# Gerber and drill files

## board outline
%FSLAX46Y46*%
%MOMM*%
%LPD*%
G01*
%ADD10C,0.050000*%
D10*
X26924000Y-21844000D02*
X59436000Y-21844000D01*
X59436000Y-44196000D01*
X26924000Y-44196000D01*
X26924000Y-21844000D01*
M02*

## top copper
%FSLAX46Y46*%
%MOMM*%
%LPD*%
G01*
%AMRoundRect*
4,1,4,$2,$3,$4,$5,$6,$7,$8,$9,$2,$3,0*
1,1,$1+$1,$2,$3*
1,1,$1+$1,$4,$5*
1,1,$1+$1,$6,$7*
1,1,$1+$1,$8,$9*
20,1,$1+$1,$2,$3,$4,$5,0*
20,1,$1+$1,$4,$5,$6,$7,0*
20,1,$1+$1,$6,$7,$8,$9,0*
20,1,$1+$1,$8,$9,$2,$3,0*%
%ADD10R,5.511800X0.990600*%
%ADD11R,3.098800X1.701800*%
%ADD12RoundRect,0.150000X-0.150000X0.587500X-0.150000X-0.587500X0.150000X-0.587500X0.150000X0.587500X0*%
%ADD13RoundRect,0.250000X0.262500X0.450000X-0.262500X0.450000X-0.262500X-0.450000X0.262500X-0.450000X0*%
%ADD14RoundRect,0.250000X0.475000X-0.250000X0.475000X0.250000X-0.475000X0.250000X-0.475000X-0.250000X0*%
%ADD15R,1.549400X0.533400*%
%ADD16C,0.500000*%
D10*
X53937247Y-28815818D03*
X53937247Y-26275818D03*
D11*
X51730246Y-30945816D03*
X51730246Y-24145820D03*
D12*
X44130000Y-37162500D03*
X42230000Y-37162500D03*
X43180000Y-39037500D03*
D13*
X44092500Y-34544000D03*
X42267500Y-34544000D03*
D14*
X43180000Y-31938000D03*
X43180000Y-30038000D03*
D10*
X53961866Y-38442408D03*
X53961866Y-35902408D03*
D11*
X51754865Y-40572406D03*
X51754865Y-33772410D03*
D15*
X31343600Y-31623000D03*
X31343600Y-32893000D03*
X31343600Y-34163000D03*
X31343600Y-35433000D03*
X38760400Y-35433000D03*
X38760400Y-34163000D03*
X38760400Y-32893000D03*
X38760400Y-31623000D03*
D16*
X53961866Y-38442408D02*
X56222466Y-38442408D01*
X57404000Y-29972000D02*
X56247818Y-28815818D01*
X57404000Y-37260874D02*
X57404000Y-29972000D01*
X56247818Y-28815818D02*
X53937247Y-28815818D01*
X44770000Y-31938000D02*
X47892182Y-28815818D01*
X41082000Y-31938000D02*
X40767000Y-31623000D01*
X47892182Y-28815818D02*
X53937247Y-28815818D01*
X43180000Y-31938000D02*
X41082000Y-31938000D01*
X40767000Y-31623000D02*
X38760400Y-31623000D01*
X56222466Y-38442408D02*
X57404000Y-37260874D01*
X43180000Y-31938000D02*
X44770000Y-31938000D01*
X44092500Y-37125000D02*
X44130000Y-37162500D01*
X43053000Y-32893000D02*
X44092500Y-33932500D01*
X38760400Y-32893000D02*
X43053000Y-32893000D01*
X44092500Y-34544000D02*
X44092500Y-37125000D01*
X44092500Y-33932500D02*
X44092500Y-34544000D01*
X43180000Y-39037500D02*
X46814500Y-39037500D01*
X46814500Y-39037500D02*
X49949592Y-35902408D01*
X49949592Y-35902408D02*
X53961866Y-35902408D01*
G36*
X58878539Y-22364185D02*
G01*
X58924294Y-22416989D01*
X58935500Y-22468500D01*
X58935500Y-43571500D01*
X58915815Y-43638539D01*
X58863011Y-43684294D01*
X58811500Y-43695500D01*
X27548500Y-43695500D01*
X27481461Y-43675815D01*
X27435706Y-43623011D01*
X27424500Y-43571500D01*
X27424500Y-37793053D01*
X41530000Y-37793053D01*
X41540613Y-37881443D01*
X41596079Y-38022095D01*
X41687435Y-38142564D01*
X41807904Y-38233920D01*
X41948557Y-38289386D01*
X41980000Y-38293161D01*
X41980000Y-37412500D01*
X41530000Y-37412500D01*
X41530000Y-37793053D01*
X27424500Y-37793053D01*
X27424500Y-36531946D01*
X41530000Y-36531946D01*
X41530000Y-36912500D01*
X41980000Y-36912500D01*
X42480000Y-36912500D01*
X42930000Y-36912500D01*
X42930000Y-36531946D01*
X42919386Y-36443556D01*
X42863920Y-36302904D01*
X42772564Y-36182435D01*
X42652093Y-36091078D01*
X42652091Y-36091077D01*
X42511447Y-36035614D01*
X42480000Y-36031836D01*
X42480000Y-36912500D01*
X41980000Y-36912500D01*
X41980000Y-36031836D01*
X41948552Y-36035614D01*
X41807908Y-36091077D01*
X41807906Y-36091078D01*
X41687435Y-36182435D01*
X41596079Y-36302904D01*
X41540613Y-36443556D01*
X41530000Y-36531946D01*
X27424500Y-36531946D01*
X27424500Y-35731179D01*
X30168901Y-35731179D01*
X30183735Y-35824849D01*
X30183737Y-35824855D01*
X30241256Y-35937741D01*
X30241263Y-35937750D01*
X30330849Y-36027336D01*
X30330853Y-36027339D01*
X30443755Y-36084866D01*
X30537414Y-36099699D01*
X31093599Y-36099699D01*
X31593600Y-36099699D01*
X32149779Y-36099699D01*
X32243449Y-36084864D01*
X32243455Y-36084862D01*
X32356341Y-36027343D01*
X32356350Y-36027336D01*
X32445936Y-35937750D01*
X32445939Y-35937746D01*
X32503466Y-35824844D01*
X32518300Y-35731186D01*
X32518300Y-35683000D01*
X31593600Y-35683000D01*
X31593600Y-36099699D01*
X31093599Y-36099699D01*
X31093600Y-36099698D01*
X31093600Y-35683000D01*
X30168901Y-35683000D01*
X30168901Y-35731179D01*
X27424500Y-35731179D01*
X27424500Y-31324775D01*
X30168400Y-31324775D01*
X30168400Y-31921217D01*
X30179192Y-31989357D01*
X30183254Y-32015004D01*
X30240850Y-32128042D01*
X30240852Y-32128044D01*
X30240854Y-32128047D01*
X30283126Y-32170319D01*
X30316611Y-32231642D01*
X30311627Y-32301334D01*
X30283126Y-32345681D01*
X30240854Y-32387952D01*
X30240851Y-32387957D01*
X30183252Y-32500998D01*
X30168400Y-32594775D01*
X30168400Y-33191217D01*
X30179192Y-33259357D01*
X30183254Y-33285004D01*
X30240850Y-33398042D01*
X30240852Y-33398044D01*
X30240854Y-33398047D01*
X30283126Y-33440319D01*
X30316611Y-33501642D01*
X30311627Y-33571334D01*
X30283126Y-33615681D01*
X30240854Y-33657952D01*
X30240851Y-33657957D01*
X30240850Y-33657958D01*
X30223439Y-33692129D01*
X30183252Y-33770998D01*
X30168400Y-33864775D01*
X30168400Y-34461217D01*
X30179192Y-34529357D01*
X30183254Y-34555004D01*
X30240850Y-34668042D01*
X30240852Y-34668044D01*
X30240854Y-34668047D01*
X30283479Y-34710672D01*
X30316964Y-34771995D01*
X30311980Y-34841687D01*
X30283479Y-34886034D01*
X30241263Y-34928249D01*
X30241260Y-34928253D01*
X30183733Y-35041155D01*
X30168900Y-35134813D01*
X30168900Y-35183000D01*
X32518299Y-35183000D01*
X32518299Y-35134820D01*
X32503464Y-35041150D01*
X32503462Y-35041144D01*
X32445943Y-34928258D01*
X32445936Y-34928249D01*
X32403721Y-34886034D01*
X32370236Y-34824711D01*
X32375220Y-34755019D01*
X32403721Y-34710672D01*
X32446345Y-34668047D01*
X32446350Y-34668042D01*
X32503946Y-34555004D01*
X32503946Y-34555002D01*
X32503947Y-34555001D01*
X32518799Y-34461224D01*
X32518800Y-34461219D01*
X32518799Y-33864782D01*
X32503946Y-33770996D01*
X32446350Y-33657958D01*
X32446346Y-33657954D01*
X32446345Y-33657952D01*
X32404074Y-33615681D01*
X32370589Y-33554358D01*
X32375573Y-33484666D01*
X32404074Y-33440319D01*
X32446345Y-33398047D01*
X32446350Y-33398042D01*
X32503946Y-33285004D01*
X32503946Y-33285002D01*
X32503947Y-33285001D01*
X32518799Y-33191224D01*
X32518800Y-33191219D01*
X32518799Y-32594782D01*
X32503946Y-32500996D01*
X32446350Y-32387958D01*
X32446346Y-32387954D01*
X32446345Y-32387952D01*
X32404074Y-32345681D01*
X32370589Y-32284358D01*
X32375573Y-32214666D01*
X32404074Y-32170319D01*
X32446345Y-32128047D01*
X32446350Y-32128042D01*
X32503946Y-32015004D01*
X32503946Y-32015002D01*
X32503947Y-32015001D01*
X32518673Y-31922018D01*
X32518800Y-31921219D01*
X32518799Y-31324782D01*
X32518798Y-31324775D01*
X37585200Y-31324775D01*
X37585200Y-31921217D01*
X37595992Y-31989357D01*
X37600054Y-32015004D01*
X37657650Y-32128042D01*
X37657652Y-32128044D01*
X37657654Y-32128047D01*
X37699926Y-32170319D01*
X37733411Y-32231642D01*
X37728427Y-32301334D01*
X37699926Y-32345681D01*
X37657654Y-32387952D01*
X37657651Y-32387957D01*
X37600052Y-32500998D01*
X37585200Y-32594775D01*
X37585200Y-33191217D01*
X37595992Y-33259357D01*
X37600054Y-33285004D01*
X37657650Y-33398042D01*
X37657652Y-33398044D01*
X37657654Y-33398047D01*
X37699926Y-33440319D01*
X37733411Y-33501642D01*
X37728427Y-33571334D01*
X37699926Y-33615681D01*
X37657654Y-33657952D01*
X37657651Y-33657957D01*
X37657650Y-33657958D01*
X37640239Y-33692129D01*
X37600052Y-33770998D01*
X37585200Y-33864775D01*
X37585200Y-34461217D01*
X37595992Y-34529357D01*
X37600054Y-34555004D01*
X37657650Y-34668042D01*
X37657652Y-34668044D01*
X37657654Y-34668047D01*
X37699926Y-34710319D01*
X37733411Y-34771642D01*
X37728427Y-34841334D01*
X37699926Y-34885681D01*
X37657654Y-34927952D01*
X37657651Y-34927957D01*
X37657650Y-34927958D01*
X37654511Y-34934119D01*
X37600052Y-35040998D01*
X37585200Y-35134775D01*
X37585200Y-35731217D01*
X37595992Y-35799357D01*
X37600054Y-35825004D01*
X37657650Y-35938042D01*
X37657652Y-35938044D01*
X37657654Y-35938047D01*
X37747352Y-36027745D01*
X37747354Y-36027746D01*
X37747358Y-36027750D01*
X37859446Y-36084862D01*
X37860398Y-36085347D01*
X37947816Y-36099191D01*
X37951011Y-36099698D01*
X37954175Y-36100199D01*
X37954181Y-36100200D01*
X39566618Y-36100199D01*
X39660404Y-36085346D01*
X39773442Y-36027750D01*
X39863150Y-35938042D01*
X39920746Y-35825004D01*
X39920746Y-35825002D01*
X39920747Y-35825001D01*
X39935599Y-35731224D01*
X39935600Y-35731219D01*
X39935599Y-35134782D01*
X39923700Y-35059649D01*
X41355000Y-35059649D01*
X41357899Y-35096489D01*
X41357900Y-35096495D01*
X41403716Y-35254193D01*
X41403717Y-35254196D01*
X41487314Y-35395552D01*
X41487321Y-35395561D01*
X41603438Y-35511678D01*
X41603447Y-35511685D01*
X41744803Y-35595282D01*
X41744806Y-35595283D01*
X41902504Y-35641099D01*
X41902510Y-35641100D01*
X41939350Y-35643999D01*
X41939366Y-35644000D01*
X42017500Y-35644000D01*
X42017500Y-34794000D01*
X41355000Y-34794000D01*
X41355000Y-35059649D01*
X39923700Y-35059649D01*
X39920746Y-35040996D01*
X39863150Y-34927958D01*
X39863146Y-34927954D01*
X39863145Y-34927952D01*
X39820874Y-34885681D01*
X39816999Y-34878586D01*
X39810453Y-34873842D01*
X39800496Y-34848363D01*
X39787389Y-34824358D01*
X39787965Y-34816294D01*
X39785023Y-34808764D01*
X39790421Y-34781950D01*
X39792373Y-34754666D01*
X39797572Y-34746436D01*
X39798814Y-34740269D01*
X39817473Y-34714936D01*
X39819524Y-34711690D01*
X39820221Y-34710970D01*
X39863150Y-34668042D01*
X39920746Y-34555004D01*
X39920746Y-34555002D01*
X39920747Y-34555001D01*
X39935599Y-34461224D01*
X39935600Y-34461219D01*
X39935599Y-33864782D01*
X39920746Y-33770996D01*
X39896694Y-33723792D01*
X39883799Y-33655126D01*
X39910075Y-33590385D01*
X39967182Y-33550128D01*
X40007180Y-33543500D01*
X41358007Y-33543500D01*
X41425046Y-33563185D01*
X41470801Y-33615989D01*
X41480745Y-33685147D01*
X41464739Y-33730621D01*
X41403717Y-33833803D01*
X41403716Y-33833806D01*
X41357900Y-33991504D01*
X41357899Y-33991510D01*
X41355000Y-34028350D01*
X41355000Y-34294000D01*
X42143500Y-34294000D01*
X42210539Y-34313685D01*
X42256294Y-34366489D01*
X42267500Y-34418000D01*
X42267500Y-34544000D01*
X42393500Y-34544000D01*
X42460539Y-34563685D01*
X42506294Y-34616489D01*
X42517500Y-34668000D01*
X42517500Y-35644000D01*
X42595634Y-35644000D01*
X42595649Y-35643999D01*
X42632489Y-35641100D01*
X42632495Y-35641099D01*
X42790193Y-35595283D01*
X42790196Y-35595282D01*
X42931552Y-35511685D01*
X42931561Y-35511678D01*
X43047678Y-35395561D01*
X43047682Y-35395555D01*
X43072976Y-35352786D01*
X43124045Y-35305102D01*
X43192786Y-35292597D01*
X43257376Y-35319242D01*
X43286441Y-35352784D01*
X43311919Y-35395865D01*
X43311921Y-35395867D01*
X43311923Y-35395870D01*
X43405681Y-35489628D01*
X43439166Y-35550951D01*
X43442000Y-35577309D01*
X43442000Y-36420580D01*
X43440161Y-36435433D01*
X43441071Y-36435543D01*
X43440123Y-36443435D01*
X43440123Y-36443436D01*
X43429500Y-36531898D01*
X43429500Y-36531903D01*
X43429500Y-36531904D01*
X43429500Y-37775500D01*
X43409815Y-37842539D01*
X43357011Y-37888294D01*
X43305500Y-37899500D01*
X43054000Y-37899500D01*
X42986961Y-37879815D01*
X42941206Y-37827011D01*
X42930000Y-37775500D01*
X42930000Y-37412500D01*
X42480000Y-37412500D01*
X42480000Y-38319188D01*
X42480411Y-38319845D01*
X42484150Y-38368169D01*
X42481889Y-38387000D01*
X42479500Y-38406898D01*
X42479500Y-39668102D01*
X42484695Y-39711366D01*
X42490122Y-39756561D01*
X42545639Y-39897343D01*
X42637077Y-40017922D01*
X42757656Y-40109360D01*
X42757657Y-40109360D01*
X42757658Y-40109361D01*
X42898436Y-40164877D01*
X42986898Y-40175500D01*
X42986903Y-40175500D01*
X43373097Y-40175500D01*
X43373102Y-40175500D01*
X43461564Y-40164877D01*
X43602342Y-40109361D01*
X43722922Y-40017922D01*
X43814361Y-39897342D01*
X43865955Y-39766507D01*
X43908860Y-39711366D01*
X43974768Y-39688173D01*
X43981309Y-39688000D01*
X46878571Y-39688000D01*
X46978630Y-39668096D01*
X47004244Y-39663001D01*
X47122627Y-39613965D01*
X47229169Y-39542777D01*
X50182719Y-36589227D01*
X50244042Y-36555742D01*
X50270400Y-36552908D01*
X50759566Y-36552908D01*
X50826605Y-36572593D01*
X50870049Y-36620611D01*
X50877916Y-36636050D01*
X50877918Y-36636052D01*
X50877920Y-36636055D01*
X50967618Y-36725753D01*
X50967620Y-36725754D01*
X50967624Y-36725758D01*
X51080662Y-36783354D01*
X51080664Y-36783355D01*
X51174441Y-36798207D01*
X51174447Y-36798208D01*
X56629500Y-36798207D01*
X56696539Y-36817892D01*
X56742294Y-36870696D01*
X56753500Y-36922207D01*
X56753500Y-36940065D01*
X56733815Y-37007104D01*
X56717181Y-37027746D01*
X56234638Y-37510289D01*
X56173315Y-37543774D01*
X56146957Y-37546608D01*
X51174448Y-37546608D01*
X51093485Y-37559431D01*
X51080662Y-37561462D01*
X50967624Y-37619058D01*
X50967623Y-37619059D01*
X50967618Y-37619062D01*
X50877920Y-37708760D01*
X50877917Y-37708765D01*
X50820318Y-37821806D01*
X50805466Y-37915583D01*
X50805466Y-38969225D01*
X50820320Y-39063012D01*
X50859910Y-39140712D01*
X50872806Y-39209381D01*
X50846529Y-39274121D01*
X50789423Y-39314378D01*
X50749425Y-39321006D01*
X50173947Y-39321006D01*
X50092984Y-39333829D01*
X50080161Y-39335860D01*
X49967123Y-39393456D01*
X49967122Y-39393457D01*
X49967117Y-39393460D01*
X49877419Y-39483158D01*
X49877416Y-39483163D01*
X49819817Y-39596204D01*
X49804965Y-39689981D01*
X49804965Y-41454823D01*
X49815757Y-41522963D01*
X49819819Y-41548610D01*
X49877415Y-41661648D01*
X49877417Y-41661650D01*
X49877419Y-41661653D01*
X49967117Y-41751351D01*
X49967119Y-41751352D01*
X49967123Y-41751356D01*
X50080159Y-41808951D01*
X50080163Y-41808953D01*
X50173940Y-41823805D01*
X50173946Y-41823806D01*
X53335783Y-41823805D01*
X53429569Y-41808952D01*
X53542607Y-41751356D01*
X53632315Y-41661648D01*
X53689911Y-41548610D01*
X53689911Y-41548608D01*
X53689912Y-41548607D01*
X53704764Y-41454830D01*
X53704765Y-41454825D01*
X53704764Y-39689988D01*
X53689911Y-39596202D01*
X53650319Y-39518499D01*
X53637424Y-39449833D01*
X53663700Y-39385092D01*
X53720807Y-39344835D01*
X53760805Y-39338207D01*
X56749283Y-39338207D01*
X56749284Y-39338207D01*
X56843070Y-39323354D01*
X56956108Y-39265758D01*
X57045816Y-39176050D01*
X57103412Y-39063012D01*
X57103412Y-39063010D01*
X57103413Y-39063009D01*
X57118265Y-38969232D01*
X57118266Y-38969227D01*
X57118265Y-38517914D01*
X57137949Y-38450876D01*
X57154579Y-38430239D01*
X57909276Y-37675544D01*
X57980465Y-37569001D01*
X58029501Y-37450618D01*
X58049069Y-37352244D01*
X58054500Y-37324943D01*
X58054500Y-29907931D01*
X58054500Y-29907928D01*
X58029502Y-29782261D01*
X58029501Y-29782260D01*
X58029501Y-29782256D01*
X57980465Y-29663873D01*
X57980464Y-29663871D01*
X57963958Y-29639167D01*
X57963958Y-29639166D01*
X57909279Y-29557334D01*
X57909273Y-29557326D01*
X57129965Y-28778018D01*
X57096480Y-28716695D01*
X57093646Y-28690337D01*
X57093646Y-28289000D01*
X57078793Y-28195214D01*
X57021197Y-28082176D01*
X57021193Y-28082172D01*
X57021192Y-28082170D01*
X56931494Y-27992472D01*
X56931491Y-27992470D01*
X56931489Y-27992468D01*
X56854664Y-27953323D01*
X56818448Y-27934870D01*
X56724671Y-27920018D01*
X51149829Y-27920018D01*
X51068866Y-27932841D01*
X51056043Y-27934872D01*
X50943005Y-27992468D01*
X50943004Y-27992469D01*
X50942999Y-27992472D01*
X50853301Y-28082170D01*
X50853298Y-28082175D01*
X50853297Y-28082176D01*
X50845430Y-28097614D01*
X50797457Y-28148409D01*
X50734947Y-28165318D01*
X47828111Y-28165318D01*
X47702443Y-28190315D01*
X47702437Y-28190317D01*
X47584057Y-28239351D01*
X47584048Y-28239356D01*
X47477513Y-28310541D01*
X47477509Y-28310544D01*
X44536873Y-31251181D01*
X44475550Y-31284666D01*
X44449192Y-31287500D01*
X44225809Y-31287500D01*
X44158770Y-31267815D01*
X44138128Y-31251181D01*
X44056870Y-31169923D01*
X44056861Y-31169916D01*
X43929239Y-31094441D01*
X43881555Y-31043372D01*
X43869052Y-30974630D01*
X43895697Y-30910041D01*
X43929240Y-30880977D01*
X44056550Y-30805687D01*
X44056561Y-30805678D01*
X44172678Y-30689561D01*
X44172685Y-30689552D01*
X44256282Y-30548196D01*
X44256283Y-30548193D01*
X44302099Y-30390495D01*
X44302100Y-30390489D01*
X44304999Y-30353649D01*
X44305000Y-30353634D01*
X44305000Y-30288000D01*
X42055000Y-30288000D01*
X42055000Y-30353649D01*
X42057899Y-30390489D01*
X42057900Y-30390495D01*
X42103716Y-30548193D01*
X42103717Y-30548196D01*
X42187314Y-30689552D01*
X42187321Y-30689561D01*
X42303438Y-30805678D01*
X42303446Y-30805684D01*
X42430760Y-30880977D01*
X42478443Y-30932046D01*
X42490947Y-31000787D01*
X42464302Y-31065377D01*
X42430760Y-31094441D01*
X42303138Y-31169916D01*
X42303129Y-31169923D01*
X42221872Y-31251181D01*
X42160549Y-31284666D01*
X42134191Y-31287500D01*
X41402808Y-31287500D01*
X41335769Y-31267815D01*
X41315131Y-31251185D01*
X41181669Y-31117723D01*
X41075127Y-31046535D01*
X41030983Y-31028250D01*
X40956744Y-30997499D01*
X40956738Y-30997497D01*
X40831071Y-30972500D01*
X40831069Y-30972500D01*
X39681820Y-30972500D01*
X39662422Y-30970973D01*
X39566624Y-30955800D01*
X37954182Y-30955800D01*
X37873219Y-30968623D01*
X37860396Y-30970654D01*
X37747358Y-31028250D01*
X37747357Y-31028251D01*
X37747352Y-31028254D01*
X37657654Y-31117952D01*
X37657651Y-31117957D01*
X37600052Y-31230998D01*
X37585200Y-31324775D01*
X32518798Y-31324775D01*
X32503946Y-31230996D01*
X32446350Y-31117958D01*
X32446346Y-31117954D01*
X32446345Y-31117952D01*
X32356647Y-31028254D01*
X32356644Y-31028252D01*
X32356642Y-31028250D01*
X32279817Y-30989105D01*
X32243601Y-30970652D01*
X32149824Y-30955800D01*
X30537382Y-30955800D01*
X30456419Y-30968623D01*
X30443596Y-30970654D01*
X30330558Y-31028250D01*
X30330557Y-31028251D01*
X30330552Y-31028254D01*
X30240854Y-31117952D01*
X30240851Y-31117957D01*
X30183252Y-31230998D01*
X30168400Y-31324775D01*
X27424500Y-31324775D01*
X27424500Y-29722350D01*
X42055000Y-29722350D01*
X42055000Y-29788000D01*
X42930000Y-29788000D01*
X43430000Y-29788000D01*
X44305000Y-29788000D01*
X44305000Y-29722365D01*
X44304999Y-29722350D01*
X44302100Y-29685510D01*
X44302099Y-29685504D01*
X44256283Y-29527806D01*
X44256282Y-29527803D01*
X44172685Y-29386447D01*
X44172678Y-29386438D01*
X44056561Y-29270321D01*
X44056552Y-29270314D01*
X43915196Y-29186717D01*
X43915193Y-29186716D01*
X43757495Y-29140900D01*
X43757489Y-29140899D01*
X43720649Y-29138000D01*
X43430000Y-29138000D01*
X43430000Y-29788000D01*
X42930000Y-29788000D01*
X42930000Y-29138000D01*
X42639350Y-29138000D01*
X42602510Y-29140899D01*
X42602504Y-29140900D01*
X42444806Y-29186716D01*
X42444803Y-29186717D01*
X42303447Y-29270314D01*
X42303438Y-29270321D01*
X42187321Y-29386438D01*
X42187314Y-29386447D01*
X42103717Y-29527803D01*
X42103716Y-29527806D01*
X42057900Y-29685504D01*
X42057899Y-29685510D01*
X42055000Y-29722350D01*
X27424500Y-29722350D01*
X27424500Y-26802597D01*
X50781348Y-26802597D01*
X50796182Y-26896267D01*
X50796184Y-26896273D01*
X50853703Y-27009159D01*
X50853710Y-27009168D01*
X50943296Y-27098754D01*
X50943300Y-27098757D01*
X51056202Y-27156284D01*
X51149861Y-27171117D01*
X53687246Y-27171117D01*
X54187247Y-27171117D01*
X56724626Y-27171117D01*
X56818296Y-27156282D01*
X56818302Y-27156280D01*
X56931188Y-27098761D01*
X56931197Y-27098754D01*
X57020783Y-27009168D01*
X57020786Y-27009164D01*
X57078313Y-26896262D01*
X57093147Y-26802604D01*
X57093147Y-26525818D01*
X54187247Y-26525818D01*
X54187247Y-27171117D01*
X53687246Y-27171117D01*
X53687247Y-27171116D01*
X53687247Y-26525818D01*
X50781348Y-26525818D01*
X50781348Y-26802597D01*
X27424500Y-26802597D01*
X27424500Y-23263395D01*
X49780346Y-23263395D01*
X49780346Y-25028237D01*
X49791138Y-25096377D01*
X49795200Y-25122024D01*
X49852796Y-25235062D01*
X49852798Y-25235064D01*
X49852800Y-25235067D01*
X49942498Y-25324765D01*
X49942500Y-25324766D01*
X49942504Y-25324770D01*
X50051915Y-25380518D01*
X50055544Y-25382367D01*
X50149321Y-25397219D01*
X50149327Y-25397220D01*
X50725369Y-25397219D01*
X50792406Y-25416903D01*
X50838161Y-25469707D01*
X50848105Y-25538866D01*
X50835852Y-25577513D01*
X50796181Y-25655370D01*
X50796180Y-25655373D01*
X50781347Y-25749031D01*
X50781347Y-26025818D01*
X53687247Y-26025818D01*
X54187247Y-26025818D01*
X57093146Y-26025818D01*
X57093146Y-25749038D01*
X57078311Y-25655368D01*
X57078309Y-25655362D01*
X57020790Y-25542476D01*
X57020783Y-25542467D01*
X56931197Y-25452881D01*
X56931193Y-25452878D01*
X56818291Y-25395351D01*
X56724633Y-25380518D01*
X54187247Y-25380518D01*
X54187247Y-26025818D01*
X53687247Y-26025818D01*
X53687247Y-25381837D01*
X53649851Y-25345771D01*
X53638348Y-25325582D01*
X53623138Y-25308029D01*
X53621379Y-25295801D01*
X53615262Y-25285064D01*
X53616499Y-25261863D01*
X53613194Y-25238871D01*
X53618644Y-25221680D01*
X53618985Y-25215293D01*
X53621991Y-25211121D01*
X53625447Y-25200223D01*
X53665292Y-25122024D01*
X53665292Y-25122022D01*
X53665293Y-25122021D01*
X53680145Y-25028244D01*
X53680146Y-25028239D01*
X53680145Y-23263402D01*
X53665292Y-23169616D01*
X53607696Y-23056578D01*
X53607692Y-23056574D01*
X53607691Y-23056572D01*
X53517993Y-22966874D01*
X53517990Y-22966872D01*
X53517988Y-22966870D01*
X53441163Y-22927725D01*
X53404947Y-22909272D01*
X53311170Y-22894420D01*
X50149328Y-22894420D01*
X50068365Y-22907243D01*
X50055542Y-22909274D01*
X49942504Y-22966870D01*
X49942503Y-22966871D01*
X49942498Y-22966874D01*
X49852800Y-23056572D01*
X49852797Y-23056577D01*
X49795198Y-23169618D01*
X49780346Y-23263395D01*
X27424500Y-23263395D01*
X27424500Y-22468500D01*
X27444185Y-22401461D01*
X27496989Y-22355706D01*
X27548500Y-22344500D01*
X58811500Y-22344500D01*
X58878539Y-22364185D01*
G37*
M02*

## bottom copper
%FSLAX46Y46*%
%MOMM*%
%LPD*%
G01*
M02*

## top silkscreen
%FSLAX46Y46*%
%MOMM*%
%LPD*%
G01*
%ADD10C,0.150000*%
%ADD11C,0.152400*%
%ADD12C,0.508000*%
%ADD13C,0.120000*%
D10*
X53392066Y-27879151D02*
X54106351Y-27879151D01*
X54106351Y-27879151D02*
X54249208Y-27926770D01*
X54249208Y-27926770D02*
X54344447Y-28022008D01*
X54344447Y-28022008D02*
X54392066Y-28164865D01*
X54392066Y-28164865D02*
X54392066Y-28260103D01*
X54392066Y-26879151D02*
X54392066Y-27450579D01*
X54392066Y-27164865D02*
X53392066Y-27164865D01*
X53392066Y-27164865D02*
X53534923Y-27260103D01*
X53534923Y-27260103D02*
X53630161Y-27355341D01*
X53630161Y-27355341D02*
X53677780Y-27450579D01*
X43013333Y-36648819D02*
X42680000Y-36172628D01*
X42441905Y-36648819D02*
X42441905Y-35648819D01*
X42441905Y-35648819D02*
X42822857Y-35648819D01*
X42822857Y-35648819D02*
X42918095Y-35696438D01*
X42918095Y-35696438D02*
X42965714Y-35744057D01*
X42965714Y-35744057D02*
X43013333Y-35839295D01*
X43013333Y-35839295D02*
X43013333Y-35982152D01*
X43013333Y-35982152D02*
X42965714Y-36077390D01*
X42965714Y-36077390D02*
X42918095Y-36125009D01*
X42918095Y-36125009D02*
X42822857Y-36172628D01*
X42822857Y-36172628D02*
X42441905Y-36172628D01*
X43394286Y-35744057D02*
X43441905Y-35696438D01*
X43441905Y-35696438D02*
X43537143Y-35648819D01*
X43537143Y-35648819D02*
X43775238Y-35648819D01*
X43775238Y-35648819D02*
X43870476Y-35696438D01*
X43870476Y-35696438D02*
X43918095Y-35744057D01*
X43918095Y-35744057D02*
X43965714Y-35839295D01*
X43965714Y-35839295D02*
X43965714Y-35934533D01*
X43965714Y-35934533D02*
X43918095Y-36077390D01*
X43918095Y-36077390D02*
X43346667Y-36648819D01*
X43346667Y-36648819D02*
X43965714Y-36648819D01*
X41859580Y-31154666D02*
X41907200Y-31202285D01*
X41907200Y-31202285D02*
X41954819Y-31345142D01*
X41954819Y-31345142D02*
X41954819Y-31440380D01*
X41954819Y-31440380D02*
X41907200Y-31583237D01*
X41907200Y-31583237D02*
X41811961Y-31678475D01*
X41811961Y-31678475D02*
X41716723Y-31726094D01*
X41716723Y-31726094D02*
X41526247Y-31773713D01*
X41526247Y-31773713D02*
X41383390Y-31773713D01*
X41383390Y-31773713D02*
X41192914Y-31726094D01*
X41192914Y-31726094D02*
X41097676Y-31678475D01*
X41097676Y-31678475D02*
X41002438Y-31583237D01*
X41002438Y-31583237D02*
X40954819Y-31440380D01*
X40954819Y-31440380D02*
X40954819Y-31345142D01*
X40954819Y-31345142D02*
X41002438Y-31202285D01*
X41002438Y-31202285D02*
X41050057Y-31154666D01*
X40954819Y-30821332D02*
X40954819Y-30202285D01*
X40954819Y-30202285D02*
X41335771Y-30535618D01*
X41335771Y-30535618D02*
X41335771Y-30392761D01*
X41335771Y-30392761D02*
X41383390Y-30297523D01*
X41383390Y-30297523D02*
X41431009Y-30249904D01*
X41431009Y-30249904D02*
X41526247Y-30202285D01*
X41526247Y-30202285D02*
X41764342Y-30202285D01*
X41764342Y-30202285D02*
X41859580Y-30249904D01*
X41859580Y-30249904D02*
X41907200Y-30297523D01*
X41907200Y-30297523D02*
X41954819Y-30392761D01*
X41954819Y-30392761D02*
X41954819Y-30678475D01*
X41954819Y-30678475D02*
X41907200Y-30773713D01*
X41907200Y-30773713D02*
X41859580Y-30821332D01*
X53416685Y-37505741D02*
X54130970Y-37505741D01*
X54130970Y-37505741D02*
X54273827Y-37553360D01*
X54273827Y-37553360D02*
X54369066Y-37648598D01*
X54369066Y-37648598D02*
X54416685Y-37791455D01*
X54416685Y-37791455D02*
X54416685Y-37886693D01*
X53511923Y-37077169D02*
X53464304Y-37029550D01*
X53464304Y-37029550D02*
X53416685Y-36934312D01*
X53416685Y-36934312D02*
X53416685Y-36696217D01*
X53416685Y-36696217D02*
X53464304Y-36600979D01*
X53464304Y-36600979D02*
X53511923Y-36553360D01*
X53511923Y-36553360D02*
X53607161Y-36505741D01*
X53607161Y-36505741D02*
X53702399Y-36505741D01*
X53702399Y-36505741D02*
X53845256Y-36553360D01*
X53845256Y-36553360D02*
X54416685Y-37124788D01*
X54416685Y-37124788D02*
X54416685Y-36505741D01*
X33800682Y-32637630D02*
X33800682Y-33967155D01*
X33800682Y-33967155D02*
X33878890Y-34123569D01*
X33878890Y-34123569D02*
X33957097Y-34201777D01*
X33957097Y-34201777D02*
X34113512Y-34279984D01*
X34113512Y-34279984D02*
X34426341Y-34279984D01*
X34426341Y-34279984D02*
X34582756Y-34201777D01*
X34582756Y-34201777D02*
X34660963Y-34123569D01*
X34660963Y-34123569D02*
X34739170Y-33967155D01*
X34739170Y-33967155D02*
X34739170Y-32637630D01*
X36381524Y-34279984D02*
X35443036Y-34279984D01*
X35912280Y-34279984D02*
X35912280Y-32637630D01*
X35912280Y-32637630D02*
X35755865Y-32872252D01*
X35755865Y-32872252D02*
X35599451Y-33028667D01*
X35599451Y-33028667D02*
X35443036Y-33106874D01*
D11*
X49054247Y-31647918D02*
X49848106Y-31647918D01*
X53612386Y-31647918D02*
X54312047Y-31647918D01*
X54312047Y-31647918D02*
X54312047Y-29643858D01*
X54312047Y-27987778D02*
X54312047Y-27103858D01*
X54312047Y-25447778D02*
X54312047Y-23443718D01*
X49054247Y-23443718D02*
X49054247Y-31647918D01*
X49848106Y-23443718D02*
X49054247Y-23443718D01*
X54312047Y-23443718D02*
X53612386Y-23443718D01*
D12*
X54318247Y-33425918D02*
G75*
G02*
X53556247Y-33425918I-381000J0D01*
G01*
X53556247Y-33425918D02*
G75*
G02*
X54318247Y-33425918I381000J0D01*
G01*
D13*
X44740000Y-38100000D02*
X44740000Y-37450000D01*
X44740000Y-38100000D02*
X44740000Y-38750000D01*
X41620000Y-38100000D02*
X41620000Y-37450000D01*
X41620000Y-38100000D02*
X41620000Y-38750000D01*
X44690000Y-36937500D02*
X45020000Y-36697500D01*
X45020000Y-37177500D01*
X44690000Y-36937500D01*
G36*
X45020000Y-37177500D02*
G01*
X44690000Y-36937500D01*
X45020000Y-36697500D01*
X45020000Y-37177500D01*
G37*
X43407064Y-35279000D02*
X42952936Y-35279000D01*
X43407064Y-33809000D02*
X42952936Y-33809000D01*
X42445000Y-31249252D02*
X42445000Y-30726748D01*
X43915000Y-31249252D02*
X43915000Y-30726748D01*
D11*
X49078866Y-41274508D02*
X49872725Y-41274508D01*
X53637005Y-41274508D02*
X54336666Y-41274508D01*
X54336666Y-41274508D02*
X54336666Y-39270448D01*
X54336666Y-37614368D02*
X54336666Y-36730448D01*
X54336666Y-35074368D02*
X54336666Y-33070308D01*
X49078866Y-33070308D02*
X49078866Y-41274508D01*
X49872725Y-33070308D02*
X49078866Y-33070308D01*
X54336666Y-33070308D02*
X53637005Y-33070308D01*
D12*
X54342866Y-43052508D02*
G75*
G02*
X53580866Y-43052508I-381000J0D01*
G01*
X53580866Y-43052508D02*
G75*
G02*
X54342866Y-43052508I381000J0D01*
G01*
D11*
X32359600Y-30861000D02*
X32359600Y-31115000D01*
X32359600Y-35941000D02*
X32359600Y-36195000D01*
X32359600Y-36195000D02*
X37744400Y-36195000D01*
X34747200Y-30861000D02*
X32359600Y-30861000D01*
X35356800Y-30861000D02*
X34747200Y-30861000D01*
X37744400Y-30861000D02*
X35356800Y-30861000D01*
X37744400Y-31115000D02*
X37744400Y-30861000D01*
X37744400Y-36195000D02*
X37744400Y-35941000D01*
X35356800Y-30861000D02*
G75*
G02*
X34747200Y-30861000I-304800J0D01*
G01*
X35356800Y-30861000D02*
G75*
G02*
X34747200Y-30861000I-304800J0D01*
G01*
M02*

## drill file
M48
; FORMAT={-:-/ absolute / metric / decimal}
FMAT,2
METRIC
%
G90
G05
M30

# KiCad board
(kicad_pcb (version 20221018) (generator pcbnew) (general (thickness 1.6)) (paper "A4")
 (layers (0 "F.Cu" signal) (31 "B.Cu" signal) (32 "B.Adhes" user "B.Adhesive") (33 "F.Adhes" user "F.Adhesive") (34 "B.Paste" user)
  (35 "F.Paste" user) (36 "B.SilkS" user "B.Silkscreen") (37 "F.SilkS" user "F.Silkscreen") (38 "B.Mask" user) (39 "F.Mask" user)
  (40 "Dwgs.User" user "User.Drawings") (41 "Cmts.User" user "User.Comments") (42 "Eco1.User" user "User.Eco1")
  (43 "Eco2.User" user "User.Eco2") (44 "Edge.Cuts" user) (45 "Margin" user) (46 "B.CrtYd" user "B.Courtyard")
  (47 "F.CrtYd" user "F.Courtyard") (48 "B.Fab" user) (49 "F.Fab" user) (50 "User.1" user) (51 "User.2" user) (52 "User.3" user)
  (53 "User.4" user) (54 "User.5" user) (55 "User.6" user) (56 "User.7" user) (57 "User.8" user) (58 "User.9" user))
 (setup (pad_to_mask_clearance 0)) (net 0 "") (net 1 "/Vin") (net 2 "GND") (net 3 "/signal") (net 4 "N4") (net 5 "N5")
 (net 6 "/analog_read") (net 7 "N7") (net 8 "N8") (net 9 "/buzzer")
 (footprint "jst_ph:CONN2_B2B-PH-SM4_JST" (layer "F.Cu") (at 51.683147 27.545818 90)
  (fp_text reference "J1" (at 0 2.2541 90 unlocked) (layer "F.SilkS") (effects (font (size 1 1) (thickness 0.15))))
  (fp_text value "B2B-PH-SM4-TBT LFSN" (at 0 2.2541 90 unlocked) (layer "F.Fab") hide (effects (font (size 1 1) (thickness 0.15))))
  (fp_line (start -4.1021 -2.6289) (end -4.1021 -1.835041) (stroke (width 0.1524) (type solid)) (layer "F.SilkS"))
  (fp_line (start -4.1021 1.929239) (end -4.1021 2.6289) (stroke (width 0.1524) (type solid)) (layer "F.SilkS"))
  (fp_line (start -4.1021 2.6289) (end -2.09804 2.6289) (stroke (width 0.1524) (type solid)) (layer "F.SilkS"))
  (fp_line (start -0.44196 2.6289) (end 0.44196 2.6289) (stroke (width 0.1524) (type solid)) (layer "F.SilkS"))
  (fp_line (start 2.09804 2.6289) (end 4.1021 2.6289) (stroke (width 0.1524) (type solid)) (layer "F.SilkS"))
  (fp_line (start 4.1021 -2.6289) (end -4.1021 -2.6289) (stroke (width 0.1524) (type solid)) (layer "F.SilkS"))
  (fp_line (start 4.1021 -1.835041) (end 4.1021 -2.6289) (stroke (width 0.1524) (type solid)) (layer "F.SilkS"))
  (fp_line (start 4.1021 2.6289) (end 4.1021 1.929239) (stroke (width 0.1524) (type solid)) (layer "F.SilkS"))
  (fp_circle (center -5.8801 2.2541) (end -5.4991 2.2541) (stroke (width 0.508) (type solid)) (fill none) (layer "F.SilkS"))
  (pad "1" smd rect (at -1.27 2.2541 90) (size 0.9906 5.5118) (layers "F.Cu" "F.Paste" "F.Mask") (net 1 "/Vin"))
  (pad "2" smd rect (at 1.27 2.2541 90) (size 0.9906 5.5118) (layers "F.Cu" "F.Paste" "F.Mask") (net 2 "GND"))
  (pad "3" smd rect (at -3.399998 0.047099 90) (size 1.7018 3.0988) (layers "F.Cu" "F.Paste" "F.Mask"))
  (pad "4" smd rect (at 3.399998 0.047099 90) (size 1.7018 3.0988) (layers "F.Cu" "F.Paste" "F.Mask")))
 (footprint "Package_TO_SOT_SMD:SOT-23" (layer "F.Cu") (at 43.18 38.1 -90)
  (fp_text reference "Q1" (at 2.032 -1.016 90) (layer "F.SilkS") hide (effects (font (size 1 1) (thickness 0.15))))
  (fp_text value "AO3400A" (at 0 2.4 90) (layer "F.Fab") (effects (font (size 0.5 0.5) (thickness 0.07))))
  (fp_line (start 0 -1.56) (end -0.65 -1.56) (stroke (width 0.12) (type solid)) (layer "F.SilkS"))
  (fp_line (start 0 -1.56) (end 0.65 -1.56) (stroke (width 0.12) (type solid)) (layer "F.SilkS"))
  (fp_line (start 0 1.56) (end -0.65 1.56) (stroke (width 0.12) (type solid)) (layer "F.SilkS"))
  (fp_line (start 0 1.56) (end 0.65 1.56) (stroke (width 0.12) (type solid)) (layer "F.SilkS"))
  (fp_poly
   (pts (xy -1.1625 -1.51) (xy -1.4025 -1.84) (xy -0.9225 -1.84) (xy -1.1625 -1.51)) (stroke (width 0.12) (type solid)) (fill solid)
   (layer "F.SilkS"))
  (pad "1" smd roundrect (at -0.9375 -0.95 270) (size 1.475 0.6) (layers "F.Cu" "F.Paste" "F.Mask") (roundrect_rratio 0.25)
   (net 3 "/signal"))
  (pad "2" smd roundrect (at -0.9375 0.95 270) (size 1.475 0.6) (layers "F.Cu" "F.Paste" "F.Mask") (roundrect_rratio 0.25) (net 2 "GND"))
  (pad "3" smd roundrect (at 0.9375 0 270) (size 1.475 0.6) (layers "F.Cu" "F.Paste" "F.Mask") (roundrect_rratio 0.25) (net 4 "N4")))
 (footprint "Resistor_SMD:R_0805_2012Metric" (layer "F.Cu") (at 43.18 34.544 180)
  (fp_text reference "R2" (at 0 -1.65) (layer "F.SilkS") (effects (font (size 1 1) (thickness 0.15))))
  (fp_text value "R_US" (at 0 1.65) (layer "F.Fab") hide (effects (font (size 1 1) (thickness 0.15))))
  (fp_line (start -0.227064 -0.735) (end 0.227064 -0.735) (stroke (width 0.12) (type solid)) (layer "F.SilkS"))
  (fp_line (start -0.227064 0.735) (end 0.227064 0.735) (stroke (width 0.12) (type solid)) (layer "F.SilkS"))
  (pad "1" smd roundrect (at -0.9125 0 180) (size 1.025 1.4) (layers "F.Cu" "F.Paste" "F.Mask") (roundrect_rratio 0.243902)
   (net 3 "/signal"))
  (pad "2" smd roundrect (at 0.9125 0 180) (size 1.025 1.4) (layers "F.Cu" "F.Paste" "F.Mask") (roundrect_rratio 0.243902) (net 2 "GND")))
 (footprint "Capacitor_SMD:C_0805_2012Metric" (layer "F.Cu") (at 43.18 30.988 90)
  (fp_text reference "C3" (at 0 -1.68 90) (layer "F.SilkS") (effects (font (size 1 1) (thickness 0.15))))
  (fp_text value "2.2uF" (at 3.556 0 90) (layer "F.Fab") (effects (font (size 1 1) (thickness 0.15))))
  (fp_line (start -0.261252 -0.735) (end 0.261252 -0.735) (stroke (width 0.12) (type solid)) (layer "F.SilkS"))
  (fp_line (start -0.261252 0.735) (end 0.261252 0.735) (stroke (width 0.12) (type solid)) (layer "F.SilkS"))
  (pad "1" smd roundrect (at -0.95 0 90) (size 1 1.45) (layers "F.Cu" "F.Paste" "F.Mask") (roundrect_rratio 0.25) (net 1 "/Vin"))
  (pad "2" smd roundrect (at 0.95 0 90) (size 1 1.45) (layers "F.Cu" "F.Paste" "F.Mask") (roundrect_rratio 0.25) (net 2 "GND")))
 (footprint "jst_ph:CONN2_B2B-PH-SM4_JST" (layer "F.Cu") (at 51.707766 37.172408 90)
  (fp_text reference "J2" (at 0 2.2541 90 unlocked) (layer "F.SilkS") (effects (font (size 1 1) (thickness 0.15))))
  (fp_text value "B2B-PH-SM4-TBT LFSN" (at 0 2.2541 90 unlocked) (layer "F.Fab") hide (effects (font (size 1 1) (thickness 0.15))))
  (fp_line (start -4.1021 -2.6289) (end -4.1021 -1.835041) (stroke (width 0.1524) (type solid)) (layer "F.SilkS"))
  (fp_line (start -4.1021 1.929239) (end -4.1021 2.6289) (stroke (width 0.1524) (type solid)) (layer "F.SilkS"))
  (fp_line (start -4.1021 2.6289) (end -2.09804 2.6289) (stroke (width 0.1524) (type solid)) (layer "F.SilkS"))
  (fp_line (start -0.44196 2.6289) (end 0.44196 2.6289) (stroke (width 0.1524) (type solid)) (layer "F.SilkS"))
  (fp_line (start 2.09804 2.6289) (end 4.1021 2.6289) (stroke (width 0.1524) (type solid)) (layer "F.SilkS"))
  (fp_line (start 4.1021 -2.6289) (end -4.1021 -2.6289) (stroke (width 0.1524) (type solid)) (layer "F.SilkS"))
  (fp_line (start 4.1021 -1.835041) (end 4.1021 -2.6289) (stroke (width 0.1524) (type solid)) (layer "F.SilkS"))
  (fp_line (start 4.1021 2.6289) (end 4.1021 1.929239) (stroke (width 0.1524) (type solid)) (layer "F.SilkS"))
  (fp_circle (center -5.8801 2.2541) (end -5.4991 2.2541) (stroke (width 0.508) (type solid)) (fill none) (layer "F.SilkS"))
  (pad "1" smd rect (at -1.27 2.2541 90) (size 0.9906 5.5118) (layers "F.Cu" "F.Paste" "F.Mask") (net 1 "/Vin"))
  (pad "2" smd rect (at 1.27 2.2541 90) (size 0.9906 5.5118) (layers "F.Cu" "F.Paste" "F.Mask") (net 4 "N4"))
  (pad "3" smd rect (at -3.399998 0.047099 90) (size 1.7018 3.0988) (layers "F.Cu" "F.Paste" "F.Mask"))
  (pad "4" smd rect (at 3.399998 0.047099 90) (size 1.7018 3.0988) (layers "F.Cu" "F.Paste" "F.Mask")))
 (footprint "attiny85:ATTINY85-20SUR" (layer "F.Cu") (at 35.052 33.528)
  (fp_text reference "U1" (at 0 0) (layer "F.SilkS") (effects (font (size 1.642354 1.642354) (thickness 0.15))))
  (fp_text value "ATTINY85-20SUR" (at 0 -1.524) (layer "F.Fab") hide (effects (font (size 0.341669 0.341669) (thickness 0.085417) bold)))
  (fp_line (start -2.6924 -2.667) (end -2.6924 -2.413) (stroke (width 0.1524) (type solid)) (layer "F.SilkS"))
  (fp_line (start -2.6924 2.413) (end -2.6924 2.667) (stroke (width 0.1524) (type solid)) (layer "F.SilkS"))
  (fp_line (start -2.6924 2.667) (end 2.6924 2.667) (stroke (width 0.1524) (type solid)) (layer "F.SilkS"))
  (fp_line (start -0.3048 -2.667) (end -2.6924 -2.667) (stroke (width 0.1524) (type solid)) (layer "F.SilkS"))
  (fp_line (start 0.3048 -2.667) (end -0.3048 -2.667) (stroke (width 0.1524) (type solid)) (layer "F.SilkS"))
  (fp_line (start 2.6924 -2.667) (end 0.3048 -2.667) (stroke (width 0.1524) (type solid)) (layer "F.SilkS"))
  (fp_line (start 2.6924 -2.413) (end 2.6924 -2.667) (stroke (width 0.1524) (type solid)) (layer "F.SilkS"))
  (fp_line (start 2.6924 2.667) (end 2.6924 2.413) (stroke (width 0.1524) (type solid)) (layer "F.SilkS"))
  (fp_arc (start 0.3048 -2.667) (mid 0 -2.3622) (end -0.3048 -2.667) (stroke (width 0.1524) (type solid)) (layer "F.SilkS"))
  (fp_arc (start 0.3048 -2.667) (mid 0 -2.3622) (end -0.3048 -2.667) (stroke (width 0.1524) (type solid)) (layer "F.SilkS"))
  (pad "1" smd rect (at -3.7084 -1.905) (size 1.5494 0.5334) (layers "F.Cu" "F.Paste" "F.Mask") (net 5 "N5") (solder_mask_margin 0.102))
  (pad "2" smd rect (at -3.7084 -0.635) (size 1.5494 0.5334) (layers "F.Cu" "F.Paste" "F.Mask") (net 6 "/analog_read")
   (solder_mask_margin 0.102))
  (pad "3" smd rect (at -3.7084 0.635) (size 1.5494 0.5334) (layers "F.Cu" "F.Paste" "F.Mask") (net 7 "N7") (solder_mask_margin 0.102))
  (pad "4" smd rect (at -3.7084 1.905) (size 1.5494 0.5334) (layers "F.Cu" "F.Paste" "F.Mask") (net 2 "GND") (solder_mask_margin 0.102))
  (pad "5" smd rect (at 3.7084 1.905) (size 1.5494 0.5334) (layers "F.Cu" "F.Paste" "F.Mask") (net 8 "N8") (solder_mask_margin 0.102))
  (pad "6" smd rect (at 3.7084 0.635) (size 1.5494 0.5334) (layers "F.Cu" "F.Paste" "F.Mask") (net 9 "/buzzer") (solder_mask_margin 0.102))
  (pad "7" smd rect (at 3.7084 -0.635) (size 1.5494 0.5334) (layers "F.Cu" "F.Paste" "F.Mask") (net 3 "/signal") (solder_mask_margin 0.102))
  (pad "8" smd rect (at 3.7084 -1.905) (size 1.5494 0.5334) (layers "F.Cu" "F.Paste" "F.Mask") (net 1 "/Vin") (solder_mask_margin 0.102)))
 (gr_rect (start 26.924 21.844) (end 59.436 44.196) (stroke (width 0.05) (type default)) (fill none) (layer "Edge.Cuts"))
 (segment (start 53.961866 38.442408) (end 56.222466 38.442408) (width 0.5) (layer "F.Cu") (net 1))
 (segment (start 57.404 29.972) (end 56.247818 28.815818) (width 0.5) (layer "F.Cu") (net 1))
 (segment (start 57.404 37.260874) (end 57.404 29.972) (width 0.5) (layer "F.Cu") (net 1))
 (segment (start 56.247818 28.815818) (end 53.937247 28.815818) (width 0.5) (layer "F.Cu") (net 1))
 (segment (start 44.77 31.938) (end 47.892182 28.815818) (width 0.5) (layer "F.Cu") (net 1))
 (segment (start 41.082 31.938) (end 40.767 31.623) (width 0.5) (layer "F.Cu") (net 1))
 (segment (start 47.892182 28.815818) (end 53.937247 28.815818) (width 0.5) (layer "F.Cu") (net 1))
 (segment (start 43.18 31.938) (end 41.082 31.938) (width 0.5) (layer "F.Cu") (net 1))
 (segment (start 40.767 31.623) (end 38.7604 31.623) (width 0.5) (layer "F.Cu") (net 1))
 (segment (start 56.222466 38.442408) (end 57.404 37.260874) (width 0.5) (layer "F.Cu") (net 1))
 (segment (start 43.18 31.938) (end 44.77 31.938) (width 0.5) (layer "F.Cu") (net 1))
 (segment (start 44.0925 37.125) (end 44.13 37.1625) (width 0.5) (layer "F.Cu") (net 3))
 (segment (start 43.053 32.893) (end 44.0925 33.9325) (width 0.5) (layer "F.Cu") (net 3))
 (segment (start 38.7604 32.893) (end 43.053 32.893) (width 0.5) (layer "F.Cu") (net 3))
 (segment (start 44.0925 34.544) (end 44.0925 37.125) (width 0.5) (layer "F.Cu") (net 3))
 (segment (start 44.0925 33.9325) (end 44.0925 34.544) (width 0.5) (layer "F.Cu") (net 3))
 (segment (start 43.18 39.0375) (end 46.8145 39.0375) (width 0.5) (layer "F.Cu") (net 4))
 (segment (start 46.8145 39.0375) (end 49.949592 35.902408) (width 0.5) (layer "F.Cu") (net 4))
 (segment (start 49.949592 35.902408) (end 53.961866 35.902408) (width 0.5) (layer "F.Cu") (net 4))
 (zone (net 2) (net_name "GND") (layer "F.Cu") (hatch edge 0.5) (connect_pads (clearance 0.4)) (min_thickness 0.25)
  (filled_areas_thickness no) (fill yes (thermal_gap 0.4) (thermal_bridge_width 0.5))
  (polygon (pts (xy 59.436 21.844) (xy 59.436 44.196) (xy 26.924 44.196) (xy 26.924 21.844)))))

